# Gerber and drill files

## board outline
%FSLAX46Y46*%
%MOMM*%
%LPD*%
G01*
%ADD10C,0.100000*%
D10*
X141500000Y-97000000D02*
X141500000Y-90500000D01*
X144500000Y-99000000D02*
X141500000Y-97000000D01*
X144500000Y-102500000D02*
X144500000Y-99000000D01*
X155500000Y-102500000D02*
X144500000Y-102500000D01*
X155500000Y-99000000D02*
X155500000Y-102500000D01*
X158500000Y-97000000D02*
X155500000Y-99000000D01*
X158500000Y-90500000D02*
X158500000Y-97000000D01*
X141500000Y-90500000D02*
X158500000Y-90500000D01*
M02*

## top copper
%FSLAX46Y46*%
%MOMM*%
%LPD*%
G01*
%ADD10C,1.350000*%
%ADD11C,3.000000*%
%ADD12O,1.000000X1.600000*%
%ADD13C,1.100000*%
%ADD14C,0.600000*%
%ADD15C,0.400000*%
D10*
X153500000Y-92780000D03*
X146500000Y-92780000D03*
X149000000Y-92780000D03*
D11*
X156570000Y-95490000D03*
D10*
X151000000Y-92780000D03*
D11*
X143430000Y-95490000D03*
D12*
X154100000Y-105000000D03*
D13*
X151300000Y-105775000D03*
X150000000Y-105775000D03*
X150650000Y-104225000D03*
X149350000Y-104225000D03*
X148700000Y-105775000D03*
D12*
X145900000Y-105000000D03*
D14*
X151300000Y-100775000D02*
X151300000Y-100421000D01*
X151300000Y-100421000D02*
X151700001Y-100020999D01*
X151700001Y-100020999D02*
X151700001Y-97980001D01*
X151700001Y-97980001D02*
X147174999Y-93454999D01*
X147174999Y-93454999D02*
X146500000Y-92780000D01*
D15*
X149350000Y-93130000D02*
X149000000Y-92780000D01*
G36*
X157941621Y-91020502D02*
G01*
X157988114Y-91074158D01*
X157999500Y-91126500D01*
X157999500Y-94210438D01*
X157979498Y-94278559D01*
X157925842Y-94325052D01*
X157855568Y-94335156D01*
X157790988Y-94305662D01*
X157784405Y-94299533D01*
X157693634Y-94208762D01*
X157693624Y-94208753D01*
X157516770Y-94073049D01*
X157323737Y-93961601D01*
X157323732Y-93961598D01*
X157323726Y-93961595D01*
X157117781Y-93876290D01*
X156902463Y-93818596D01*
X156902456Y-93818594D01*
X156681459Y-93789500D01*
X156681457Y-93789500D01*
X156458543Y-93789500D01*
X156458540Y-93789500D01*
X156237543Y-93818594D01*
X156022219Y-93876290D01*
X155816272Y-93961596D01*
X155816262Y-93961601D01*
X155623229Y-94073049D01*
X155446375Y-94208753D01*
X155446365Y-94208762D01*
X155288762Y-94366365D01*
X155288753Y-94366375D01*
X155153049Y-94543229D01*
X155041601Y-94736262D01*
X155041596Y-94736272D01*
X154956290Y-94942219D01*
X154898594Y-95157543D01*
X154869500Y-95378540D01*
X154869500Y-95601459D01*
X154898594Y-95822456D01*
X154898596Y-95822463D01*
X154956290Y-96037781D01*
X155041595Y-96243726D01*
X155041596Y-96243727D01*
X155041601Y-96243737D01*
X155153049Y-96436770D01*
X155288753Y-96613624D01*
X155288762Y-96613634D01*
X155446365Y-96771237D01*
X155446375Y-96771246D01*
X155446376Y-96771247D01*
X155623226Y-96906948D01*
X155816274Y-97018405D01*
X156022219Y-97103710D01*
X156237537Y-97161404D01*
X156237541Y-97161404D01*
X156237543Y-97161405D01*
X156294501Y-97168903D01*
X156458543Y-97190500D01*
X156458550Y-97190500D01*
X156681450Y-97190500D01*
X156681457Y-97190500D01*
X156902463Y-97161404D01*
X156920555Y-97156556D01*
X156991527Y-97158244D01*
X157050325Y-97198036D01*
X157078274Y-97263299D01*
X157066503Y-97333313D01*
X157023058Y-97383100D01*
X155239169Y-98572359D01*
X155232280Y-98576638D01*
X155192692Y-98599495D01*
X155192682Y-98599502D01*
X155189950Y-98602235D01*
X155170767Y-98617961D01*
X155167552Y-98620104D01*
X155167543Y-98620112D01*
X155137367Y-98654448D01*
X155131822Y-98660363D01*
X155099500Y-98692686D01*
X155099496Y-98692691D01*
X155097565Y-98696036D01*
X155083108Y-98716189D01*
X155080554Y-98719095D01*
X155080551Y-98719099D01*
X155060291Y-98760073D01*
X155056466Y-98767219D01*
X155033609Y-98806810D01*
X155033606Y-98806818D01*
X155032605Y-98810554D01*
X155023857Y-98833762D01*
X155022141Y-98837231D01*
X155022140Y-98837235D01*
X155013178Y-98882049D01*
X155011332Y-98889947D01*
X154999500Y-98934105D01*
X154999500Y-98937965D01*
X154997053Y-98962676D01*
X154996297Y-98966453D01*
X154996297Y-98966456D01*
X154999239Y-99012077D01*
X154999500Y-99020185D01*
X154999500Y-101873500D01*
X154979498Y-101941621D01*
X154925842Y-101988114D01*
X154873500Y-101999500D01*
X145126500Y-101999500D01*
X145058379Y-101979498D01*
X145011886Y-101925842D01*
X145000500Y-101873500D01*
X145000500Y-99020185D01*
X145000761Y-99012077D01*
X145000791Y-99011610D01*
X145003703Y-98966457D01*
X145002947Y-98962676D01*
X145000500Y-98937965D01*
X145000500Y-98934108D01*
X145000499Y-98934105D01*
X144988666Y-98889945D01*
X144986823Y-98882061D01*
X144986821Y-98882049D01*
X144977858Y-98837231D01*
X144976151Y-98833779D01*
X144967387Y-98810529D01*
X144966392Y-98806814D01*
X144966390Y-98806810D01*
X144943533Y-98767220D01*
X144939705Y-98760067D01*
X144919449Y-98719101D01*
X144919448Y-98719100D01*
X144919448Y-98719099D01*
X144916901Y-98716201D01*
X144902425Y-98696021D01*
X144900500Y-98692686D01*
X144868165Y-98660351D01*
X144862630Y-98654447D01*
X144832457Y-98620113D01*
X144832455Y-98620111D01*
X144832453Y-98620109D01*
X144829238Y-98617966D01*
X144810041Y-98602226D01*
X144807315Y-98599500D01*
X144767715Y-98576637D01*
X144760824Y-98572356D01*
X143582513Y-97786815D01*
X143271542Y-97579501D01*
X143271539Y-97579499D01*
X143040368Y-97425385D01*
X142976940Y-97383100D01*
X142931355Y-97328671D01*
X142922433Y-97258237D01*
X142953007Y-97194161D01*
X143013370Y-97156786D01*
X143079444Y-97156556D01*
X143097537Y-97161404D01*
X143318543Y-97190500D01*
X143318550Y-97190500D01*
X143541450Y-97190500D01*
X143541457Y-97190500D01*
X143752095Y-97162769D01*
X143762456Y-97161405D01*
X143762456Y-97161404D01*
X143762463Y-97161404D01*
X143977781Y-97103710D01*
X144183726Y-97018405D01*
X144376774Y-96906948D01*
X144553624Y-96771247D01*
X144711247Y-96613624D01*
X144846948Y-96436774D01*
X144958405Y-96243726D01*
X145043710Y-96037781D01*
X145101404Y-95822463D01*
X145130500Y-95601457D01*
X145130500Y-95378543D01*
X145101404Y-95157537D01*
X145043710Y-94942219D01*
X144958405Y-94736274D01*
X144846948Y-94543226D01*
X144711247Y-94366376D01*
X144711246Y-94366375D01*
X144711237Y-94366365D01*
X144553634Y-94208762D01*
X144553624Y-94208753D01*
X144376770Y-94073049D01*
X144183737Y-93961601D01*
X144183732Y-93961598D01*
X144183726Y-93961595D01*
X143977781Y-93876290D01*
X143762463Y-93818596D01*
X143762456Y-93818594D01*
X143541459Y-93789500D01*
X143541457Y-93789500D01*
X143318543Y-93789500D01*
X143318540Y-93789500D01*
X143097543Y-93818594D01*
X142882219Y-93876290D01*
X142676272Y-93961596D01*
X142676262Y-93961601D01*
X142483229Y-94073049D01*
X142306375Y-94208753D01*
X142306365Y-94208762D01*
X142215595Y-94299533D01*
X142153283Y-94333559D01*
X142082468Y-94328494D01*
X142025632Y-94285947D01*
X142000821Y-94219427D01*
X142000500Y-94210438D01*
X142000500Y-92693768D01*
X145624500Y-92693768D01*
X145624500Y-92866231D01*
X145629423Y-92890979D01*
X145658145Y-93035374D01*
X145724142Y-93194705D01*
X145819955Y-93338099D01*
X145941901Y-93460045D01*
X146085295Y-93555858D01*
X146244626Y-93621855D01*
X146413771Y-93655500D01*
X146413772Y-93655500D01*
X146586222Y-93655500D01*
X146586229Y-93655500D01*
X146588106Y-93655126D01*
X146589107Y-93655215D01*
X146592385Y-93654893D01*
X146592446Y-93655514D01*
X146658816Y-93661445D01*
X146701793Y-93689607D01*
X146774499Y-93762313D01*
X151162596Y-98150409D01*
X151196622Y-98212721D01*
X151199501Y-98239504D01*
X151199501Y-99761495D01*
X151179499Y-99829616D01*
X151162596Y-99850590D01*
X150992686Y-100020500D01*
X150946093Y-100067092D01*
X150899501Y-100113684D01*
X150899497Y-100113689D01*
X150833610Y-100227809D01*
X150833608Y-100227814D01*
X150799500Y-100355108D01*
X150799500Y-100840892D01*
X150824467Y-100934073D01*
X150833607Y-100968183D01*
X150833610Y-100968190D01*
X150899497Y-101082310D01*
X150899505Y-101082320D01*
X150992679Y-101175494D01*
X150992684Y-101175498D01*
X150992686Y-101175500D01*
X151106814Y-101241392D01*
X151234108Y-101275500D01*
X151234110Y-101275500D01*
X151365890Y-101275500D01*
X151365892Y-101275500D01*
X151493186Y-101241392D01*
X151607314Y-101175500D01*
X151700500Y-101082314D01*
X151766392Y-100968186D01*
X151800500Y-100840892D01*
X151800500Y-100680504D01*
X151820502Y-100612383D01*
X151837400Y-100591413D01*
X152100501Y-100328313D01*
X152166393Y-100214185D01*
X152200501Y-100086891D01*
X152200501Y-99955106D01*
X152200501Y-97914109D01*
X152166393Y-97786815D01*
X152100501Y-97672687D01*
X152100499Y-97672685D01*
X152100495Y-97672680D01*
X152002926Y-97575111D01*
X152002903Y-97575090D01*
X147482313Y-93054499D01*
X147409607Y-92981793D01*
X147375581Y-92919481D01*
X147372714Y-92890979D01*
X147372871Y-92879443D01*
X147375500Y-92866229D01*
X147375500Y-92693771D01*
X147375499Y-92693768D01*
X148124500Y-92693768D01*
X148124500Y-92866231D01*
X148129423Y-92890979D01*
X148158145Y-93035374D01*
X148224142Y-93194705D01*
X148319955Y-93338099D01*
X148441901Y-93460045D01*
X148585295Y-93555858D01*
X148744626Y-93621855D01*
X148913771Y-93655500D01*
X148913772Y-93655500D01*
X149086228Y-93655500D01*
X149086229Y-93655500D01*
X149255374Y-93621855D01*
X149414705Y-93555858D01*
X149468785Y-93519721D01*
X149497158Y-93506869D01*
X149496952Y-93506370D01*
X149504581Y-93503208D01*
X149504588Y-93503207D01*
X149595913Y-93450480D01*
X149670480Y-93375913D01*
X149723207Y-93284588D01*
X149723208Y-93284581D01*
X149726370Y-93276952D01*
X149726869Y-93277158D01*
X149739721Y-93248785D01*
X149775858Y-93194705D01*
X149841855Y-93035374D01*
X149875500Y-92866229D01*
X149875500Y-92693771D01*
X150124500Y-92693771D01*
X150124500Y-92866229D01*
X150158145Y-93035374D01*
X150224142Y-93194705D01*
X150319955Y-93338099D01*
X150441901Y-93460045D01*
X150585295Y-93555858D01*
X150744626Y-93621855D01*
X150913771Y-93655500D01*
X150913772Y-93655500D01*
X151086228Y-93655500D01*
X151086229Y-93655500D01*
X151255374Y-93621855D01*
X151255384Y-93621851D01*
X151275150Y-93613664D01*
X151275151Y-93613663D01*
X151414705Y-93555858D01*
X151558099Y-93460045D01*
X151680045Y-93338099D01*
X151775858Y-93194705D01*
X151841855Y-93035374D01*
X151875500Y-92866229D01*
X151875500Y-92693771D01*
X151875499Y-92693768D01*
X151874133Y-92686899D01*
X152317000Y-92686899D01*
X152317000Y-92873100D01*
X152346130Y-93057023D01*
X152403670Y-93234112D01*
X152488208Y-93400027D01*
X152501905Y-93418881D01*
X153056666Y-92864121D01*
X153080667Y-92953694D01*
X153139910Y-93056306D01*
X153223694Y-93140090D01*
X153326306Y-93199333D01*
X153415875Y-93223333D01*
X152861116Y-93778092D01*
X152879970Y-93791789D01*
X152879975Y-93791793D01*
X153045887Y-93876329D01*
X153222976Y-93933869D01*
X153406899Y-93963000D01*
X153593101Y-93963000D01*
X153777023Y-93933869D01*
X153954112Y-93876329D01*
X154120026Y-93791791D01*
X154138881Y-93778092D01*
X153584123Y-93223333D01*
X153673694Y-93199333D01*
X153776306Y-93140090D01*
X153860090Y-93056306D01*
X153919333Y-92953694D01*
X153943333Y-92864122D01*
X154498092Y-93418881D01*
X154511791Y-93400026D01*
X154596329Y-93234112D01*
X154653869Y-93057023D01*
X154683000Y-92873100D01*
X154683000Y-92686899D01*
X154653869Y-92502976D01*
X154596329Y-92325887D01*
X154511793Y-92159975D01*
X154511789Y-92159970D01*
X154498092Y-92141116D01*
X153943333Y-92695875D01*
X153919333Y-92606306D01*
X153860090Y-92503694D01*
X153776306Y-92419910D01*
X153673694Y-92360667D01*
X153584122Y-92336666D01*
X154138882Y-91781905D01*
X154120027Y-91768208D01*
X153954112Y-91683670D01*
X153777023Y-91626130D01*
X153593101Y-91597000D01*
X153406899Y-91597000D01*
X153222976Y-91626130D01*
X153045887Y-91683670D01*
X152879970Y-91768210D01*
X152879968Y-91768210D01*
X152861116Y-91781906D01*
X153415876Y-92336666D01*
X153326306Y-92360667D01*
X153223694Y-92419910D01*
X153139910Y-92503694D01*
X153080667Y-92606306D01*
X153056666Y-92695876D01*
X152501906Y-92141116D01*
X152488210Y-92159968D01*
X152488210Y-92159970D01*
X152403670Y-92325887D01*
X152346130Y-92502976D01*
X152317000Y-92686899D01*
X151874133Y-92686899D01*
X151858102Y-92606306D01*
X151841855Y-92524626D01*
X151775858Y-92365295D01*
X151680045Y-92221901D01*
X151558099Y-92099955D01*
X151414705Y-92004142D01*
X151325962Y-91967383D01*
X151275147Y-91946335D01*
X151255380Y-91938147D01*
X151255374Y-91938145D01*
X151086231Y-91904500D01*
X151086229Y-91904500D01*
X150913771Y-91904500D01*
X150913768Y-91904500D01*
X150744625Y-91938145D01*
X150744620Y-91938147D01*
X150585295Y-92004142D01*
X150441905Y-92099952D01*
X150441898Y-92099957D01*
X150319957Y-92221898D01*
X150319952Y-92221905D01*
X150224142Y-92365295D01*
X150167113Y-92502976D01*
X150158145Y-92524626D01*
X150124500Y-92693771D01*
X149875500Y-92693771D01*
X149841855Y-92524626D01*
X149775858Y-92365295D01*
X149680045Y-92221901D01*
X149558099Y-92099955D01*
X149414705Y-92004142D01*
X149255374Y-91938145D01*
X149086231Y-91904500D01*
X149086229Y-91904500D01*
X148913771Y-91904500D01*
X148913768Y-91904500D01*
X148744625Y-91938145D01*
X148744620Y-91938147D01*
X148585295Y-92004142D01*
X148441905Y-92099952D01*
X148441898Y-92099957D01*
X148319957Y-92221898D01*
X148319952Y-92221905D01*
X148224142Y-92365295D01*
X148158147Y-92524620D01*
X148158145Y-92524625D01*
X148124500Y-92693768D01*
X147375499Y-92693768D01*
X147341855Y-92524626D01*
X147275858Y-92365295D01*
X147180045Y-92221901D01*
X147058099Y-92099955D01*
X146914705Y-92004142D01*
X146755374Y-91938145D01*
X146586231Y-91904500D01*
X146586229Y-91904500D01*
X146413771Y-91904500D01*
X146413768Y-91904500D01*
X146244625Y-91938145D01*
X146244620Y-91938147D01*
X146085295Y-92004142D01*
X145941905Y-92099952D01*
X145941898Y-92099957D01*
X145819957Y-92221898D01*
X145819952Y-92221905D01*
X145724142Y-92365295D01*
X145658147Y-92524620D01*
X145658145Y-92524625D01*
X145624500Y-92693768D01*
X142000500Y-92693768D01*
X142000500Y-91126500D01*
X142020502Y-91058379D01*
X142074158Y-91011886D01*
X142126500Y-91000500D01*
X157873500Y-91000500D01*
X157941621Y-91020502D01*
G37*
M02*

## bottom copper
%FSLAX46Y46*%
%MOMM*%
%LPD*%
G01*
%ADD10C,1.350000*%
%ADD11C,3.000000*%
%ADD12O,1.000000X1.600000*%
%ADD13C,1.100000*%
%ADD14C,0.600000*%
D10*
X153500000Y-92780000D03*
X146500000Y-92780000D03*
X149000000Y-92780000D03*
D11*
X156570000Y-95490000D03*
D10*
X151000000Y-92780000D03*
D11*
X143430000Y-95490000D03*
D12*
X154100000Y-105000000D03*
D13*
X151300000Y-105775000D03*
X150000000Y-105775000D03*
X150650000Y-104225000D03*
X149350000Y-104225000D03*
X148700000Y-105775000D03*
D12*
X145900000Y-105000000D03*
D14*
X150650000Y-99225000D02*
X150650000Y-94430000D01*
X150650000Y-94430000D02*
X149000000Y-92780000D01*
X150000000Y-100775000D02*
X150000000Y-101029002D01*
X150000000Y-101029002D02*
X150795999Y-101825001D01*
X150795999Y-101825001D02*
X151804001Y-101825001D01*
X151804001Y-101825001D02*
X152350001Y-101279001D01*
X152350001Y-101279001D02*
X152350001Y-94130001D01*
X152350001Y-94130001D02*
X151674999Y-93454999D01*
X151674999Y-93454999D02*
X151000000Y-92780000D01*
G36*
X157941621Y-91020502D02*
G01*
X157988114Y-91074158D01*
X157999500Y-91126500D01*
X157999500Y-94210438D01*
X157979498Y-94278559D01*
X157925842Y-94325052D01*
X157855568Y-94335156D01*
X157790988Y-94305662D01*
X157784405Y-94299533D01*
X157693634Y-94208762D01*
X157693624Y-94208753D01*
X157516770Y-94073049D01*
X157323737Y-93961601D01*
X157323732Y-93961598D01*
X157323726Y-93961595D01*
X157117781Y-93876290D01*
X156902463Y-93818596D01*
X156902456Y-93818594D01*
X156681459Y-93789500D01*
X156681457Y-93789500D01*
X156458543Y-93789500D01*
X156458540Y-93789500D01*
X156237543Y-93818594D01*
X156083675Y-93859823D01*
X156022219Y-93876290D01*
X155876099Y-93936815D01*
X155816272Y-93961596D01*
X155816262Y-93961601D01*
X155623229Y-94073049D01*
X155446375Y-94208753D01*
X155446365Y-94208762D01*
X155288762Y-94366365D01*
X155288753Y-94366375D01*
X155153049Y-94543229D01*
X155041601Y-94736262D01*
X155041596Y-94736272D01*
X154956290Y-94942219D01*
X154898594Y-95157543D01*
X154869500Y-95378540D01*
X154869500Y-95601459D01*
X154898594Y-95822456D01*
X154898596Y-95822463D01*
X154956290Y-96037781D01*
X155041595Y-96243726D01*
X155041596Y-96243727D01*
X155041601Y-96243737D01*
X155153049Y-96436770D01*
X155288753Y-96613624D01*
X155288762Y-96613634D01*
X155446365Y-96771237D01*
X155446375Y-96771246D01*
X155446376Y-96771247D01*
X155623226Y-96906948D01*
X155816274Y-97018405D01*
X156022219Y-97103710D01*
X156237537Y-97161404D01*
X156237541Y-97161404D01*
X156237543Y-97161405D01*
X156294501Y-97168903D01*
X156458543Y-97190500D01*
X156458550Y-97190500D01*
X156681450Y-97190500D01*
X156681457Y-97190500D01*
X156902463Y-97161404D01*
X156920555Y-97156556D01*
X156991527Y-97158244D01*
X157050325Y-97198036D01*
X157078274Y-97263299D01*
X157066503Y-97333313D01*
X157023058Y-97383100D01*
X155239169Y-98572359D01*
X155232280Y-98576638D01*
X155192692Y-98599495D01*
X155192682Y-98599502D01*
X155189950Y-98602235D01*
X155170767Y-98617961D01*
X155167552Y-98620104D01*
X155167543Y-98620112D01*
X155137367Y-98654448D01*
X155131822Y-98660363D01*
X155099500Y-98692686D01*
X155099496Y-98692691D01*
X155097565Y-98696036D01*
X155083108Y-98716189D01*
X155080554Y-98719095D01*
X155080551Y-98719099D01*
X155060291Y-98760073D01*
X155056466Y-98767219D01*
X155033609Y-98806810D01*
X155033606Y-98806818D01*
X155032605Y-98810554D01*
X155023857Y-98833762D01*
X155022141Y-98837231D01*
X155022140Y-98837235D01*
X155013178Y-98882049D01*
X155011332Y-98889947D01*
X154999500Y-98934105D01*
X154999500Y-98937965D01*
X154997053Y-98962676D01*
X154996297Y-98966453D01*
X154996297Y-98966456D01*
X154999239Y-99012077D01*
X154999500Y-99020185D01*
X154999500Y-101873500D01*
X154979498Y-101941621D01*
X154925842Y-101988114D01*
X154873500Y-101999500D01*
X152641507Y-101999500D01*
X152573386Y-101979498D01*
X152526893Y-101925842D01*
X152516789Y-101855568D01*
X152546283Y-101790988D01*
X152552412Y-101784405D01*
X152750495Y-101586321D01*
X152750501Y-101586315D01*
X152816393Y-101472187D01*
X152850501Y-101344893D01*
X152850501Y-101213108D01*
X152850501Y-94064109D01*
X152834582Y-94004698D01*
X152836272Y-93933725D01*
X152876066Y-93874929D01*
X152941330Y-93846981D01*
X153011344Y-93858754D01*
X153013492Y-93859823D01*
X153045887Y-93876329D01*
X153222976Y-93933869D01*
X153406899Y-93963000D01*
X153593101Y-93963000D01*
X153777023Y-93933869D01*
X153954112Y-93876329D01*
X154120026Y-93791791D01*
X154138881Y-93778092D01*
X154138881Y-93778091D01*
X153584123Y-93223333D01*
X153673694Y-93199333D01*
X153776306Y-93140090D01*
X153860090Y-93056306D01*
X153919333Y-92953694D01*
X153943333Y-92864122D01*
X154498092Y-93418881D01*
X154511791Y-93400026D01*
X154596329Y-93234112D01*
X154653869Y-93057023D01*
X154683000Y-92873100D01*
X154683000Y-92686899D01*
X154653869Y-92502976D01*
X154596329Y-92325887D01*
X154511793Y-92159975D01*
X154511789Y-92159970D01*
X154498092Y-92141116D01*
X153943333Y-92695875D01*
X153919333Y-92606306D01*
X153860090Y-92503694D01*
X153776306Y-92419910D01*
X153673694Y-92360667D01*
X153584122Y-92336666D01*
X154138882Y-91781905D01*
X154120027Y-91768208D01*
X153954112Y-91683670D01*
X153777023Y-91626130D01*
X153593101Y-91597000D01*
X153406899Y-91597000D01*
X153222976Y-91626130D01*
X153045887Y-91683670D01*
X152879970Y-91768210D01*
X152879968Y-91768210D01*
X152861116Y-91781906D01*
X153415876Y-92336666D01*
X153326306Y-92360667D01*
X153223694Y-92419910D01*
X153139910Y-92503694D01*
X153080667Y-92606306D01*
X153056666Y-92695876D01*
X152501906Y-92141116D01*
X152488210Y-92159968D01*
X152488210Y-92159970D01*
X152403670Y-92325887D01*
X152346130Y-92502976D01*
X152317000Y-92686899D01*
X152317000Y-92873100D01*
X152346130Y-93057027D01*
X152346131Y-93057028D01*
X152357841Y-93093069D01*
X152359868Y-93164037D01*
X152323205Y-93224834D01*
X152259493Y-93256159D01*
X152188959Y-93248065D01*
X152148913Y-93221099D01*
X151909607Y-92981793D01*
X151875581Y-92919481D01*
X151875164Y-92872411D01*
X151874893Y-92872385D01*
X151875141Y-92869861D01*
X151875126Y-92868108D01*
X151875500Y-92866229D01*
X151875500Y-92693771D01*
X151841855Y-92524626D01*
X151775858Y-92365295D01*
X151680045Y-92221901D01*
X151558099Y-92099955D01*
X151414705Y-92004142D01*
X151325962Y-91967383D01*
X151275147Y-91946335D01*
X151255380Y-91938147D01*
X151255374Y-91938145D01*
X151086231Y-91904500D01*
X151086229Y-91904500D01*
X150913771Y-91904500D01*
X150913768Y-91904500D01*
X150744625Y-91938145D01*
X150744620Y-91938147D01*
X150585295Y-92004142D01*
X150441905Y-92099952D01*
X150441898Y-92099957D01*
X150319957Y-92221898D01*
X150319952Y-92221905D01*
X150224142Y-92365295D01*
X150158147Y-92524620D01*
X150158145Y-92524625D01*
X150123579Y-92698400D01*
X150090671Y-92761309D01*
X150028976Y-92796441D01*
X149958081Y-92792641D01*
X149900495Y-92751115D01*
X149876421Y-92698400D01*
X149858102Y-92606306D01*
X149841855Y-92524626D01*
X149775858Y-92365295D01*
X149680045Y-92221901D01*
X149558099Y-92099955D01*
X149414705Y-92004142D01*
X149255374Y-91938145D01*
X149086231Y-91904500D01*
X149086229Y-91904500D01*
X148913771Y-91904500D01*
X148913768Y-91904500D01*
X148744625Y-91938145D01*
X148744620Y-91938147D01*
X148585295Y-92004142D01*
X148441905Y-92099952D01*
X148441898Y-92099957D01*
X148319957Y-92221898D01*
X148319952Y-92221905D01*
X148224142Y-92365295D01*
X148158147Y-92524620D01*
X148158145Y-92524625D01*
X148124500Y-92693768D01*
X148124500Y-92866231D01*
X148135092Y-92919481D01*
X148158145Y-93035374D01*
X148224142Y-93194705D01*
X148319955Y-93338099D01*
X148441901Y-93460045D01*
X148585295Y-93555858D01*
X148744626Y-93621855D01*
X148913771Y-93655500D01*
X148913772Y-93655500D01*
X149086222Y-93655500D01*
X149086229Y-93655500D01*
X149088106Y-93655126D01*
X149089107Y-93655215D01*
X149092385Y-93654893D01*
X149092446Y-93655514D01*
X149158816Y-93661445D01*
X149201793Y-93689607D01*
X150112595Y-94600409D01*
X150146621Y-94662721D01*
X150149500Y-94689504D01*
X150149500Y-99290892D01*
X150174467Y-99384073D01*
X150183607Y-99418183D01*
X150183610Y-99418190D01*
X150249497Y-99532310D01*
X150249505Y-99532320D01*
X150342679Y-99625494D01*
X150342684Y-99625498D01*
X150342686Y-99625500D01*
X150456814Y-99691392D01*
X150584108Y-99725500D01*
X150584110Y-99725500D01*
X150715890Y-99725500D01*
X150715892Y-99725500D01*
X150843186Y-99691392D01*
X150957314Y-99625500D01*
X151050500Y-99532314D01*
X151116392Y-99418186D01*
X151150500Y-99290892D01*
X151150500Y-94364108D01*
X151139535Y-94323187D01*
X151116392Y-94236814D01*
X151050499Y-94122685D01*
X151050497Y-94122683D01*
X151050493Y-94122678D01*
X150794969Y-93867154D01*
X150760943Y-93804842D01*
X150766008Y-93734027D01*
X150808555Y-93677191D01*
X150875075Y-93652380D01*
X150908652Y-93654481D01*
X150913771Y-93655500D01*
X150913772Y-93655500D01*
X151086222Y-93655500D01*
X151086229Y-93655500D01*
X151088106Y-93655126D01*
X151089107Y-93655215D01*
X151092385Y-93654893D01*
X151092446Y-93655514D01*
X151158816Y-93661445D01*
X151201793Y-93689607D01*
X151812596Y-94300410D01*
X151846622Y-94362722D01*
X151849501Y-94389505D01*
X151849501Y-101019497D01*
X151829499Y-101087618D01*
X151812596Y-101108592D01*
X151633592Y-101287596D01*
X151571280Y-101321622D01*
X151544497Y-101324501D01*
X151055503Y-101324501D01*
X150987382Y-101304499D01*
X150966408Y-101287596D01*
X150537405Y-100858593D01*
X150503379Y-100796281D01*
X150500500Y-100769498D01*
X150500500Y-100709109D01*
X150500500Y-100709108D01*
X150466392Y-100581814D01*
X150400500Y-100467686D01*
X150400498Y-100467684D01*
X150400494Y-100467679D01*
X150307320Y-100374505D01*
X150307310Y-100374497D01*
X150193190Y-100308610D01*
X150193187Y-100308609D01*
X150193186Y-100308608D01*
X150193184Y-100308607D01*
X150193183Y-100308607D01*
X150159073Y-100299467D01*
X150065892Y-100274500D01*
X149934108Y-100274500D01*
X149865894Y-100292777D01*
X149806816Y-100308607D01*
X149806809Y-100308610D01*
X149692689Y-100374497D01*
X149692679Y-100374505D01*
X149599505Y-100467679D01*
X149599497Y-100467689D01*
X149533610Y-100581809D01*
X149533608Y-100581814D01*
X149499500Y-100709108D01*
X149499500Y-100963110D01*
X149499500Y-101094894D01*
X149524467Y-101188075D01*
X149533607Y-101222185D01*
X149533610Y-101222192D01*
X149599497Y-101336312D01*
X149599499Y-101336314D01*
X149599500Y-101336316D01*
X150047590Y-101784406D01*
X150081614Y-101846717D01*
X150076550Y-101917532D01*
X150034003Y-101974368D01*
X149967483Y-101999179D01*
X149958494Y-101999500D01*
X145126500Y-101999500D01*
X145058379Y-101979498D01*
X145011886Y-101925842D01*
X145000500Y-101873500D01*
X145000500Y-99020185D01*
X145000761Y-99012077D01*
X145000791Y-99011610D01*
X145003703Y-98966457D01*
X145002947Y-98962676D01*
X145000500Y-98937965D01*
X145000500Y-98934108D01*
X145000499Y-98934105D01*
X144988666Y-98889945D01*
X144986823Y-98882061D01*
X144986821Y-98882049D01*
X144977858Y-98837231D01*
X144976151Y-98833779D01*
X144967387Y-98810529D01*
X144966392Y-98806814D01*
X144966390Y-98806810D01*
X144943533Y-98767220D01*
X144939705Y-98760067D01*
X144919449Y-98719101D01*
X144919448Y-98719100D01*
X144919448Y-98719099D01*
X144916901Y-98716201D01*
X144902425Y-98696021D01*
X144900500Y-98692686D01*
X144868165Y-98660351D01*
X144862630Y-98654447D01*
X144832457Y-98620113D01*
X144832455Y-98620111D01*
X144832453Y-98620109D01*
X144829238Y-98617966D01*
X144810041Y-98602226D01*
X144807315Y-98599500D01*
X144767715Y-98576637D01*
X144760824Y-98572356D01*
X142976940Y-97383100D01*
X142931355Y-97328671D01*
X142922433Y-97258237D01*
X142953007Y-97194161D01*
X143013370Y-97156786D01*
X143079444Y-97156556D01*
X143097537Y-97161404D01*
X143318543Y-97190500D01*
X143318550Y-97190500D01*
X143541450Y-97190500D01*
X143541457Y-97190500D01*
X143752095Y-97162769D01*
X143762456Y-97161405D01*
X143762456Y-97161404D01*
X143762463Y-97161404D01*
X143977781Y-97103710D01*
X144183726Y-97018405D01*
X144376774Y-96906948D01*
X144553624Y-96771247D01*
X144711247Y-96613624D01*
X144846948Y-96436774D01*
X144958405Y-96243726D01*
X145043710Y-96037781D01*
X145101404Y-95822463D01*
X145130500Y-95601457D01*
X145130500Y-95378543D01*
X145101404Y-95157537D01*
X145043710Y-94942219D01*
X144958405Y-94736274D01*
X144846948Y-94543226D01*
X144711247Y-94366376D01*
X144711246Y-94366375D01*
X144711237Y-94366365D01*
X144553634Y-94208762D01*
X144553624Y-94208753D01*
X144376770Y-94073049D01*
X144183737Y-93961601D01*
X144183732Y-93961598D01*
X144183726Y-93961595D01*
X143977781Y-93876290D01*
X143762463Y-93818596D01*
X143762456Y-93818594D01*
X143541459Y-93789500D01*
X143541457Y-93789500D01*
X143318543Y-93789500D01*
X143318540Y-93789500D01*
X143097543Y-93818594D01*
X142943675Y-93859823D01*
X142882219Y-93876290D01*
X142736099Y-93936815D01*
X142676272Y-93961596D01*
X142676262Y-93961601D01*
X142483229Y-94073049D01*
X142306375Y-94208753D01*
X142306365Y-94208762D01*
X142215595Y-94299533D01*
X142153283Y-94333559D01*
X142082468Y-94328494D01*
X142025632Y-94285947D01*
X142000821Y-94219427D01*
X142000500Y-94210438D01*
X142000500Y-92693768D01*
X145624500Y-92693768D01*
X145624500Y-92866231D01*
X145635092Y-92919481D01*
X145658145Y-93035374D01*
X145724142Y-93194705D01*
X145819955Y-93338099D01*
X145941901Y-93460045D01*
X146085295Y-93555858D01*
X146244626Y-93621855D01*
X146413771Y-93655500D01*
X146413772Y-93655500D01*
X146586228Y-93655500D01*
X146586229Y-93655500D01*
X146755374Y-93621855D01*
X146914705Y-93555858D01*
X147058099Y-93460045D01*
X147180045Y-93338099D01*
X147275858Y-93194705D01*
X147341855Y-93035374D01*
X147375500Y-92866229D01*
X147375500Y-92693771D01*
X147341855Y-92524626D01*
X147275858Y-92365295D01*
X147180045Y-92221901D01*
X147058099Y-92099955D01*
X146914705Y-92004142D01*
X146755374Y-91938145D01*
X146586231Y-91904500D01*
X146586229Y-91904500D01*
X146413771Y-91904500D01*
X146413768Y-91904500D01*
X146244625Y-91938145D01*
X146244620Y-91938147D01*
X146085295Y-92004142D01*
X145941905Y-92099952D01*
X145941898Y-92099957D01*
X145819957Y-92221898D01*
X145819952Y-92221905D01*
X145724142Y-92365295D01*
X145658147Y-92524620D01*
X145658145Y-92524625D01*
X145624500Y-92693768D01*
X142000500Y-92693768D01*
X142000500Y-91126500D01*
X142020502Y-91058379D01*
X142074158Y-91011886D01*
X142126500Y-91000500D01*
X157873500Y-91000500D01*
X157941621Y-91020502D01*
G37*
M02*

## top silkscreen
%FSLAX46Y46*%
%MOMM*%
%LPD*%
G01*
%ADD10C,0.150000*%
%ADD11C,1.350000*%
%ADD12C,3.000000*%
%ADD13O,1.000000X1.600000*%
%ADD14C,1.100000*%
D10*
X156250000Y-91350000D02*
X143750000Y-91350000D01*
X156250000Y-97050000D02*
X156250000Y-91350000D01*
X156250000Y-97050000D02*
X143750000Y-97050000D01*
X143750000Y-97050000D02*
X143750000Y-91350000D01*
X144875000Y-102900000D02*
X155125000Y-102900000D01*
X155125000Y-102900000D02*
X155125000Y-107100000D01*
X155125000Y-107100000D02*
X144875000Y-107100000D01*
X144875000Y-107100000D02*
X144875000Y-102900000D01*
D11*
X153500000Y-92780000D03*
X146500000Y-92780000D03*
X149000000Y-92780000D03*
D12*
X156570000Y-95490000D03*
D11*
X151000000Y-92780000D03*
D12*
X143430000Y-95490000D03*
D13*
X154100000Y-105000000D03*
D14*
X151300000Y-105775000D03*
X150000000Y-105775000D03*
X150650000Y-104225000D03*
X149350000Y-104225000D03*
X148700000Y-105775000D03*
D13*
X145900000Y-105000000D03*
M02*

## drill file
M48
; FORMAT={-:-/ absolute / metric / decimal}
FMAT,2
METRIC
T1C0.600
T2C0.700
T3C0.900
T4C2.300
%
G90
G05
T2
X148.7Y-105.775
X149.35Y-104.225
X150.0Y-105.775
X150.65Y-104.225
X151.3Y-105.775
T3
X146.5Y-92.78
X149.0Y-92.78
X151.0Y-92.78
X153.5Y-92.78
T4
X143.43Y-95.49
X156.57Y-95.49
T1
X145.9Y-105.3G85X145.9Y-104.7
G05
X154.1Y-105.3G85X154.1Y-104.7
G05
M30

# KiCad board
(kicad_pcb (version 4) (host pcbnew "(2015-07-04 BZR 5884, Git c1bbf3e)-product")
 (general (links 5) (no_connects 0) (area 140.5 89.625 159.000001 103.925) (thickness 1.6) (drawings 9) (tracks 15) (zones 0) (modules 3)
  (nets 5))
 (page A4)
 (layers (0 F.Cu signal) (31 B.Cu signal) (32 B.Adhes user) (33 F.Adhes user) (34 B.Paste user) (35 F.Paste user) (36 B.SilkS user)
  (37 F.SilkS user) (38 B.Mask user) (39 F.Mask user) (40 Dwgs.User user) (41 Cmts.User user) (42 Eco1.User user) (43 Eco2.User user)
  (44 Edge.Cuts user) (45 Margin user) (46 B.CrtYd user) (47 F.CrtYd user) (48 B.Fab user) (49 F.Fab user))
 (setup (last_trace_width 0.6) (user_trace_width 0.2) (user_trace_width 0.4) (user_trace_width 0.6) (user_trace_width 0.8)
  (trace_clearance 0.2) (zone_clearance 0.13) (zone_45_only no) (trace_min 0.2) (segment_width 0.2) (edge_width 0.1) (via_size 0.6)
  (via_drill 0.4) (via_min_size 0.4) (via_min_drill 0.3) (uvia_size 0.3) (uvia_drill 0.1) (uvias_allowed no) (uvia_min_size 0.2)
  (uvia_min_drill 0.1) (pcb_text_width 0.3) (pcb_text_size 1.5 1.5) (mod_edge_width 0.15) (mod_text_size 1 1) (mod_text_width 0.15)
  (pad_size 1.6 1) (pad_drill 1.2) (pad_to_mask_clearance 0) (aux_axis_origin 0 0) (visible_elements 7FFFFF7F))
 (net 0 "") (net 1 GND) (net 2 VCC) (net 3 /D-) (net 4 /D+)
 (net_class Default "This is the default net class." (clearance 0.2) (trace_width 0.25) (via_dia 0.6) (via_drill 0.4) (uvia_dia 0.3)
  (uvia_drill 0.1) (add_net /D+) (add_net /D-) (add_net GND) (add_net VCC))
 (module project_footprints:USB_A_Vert (layer F.Cu) (at 150 97)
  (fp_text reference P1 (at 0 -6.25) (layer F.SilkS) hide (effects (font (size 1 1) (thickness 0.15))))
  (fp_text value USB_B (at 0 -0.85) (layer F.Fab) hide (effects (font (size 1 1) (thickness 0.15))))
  (fp_line (start 6.25 -5.65) (end -6.25 -5.65) (layer F.SilkS) (width 0.15))
  (fp_line (start 6.25 0.05) (end 6.25 -5.65) (layer F.SilkS) (width 0.15))
  (fp_line (start 6.25 0.05) (end -6.25 0.05) (layer F.SilkS) (width 0.15))
  (fp_line (start -6.25 0.05) (end -6.25 -5.65) (layer F.SilkS) (width 0.15))
  (pad 4 thru_hole circle (at 3.5 -4.22 90) (size 1.35 1.35) (drill 0.9) (layers *.Cu *.Mask F.SilkS) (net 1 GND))
  (pad 1 thru_hole circle (at -3.5 -4.22 90) (size 1.35 1.35) (drill 0.9) (layers *.Cu *.Mask F.SilkS) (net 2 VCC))
  (pad 2 thru_hole circle (at -1 -4.22 90) (size 1.35 1.35) (drill 0.9) (layers *.Cu *.Mask F.SilkS) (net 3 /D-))
  (pad 6 thru_hole circle (at 6.57 -1.51 90) (size 3 3) (drill 2.3) (layers *.Cu *.Mask F.SilkS))
  (pad 3 thru_hole circle (at 1 -4.22 90) (size 1.35 1.35) (drill 0.9) (layers *.Cu *.Mask F.SilkS) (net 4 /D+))
  (pad 6 thru_hole circle (at -6.57 -1.51 90) (size 3 3) (drill 2.3) (layers *.Cu *.Mask F.SilkS)))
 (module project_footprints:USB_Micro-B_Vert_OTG (layer F.Cu) (at 150 105)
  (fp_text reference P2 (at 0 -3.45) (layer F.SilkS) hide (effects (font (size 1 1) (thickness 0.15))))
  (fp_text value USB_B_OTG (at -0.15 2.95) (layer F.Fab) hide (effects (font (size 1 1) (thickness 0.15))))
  (fp_line (start -5.125 -2.1) (end 5.125 -2.1) (layer F.SilkS) (width 0.15))
  (fp_line (start 5.125 -2.1) (end 5.125 2.1) (layer F.SilkS) (width 0.15))
  (fp_line (start 5.125 2.1) (end -5.125 2.1) (layer F.SilkS) (width 0.15))
  (fp_line (start -5.125 2.1) (end -5.125 -2.1) (layer F.SilkS) (width 0.15))
  (pad 6 thru_hole oval (at 4.1 0 90) (size 1.6 1) (drill oval 1.2 0.6) (layers *.Cu *.Mask F.SilkS))
  (pad 1 thru_hole circle (at 1.3 0.775 90) (size 1.1 1.1) (drill 0.7) (layers *.Cu *.Mask F.SilkS) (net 2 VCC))
  (pad 3 thru_hole circle (at 0 0.775 90) (size 1.1 1.1) (drill 0.7) (layers *.Cu *.Mask F.SilkS) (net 4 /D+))
  (pad 2 thru_hole circle (at 0.65 -0.775 90) (size 1.1 1.1) (drill 0.7) (layers *.Cu *.Mask F.SilkS) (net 3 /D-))
  (pad 4 thru_hole circle (at -0.65 -0.775 90) (size 1.1 1.1) (drill 0.7) (layers *.Cu *.Mask F.SilkS) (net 1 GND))
  (pad 5 thru_hole circle (at -1.3 0.775 90) (size 1.1 1.1) (drill 0.7) (layers *.Cu *.Mask F.SilkS) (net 1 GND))
  (pad 6 thru_hole oval (at -4.1 0 90) (size 1.6 1) (drill oval 1.2 0.6) (layers *.Cu *.Mask F.SilkS)))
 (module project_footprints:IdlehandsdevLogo (layer B.Cu) (at 150 96)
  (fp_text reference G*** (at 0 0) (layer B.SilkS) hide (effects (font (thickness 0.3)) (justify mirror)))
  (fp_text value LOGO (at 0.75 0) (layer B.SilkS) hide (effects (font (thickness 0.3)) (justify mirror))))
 (gr_line (start 141.5 97) (end 141.5 90.5) (layer Edge.Cuts) (width 0.1))
 (gr_line (start 144.5 99) (end 141.5 97) (layer Edge.Cuts) (width 0.1))
 (gr_line (start 144.5 102.5) (end 144.5 99) (layer Edge.Cuts) (width 0.1))
 (gr_line (start 155.5 102.5) (end 144.5 102.5) (layer Edge.Cuts) (width 0.1))
 (gr_line (start 155.5 99) (end 155.5 102.5) (layer Edge.Cuts) (width 0.1))
 (gr_line (start 158.5 97) (end 155.5 99) (layer Edge.Cuts) (width 0.1))
 (gr_line (start 158.5 90.5) (end 158.5 97) (layer Edge.Cuts) (width 0.1))
 (gr_line (start 141.5 90.5) (end 158.5 90.5) (layer Edge.Cuts) (width 0.1))
 (segment (start 151.3 100.775) (end 151.3 100.421) (width 0.6) (layer F.Cu) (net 2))
 (segment (start 151.3 100.421) (end 151.700001 100.020999) (width 0.6) (layer F.Cu) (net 2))
 (segment (start 151.700001 100.020999) (end 151.700001 97.980001) (width 0.6) (layer F.Cu) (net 2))
 (segment (start 151.700001 97.980001) (end 147.174999 93.454999) (width 0.6) (layer F.Cu) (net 2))
 (segment (start 147.174999 93.454999) (end 146.5 92.78) (width 0.6) (layer F.Cu) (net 2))
 (segment (start 150.65 99.225) (end 150.65 94.43) (width 0.6) (layer B.Cu) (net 3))
 (segment (start 150.65 94.43) (end 149 92.78) (width 0.6) (layer B.Cu) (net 3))
 (segment (start 149.35 93.13) (end 149 92.78) (width 0.4) (layer F.Cu) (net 3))
 (segment (start 150 100.775) (end 150 101.029002) (width 0.6) (layer B.Cu) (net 4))
 (segment (start 150 101.029002) (end 150.795999 101.825001) (width 0.6) (layer B.Cu) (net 4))
 (segment (start 150.795999 101.825001) (end 151.804001 101.825001) (width 0.6) (layer B.Cu) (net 4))
 (segment (start 151.804001 101.825001) (end 152.350001 101.279001) (width 0.6) (layer B.Cu) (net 4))
 (segment (start 152.350001 101.279001) (end 152.350001 94.130001) (width 0.6) (layer B.Cu) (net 4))
 (segment (start 152.350001 94.130001) (end 151.674999 93.454999) (width 0.6) (layer B.Cu) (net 4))
 (segment (start 151.674999 93.454999) (end 151 92.78) (width 0.6) (layer B.Cu) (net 4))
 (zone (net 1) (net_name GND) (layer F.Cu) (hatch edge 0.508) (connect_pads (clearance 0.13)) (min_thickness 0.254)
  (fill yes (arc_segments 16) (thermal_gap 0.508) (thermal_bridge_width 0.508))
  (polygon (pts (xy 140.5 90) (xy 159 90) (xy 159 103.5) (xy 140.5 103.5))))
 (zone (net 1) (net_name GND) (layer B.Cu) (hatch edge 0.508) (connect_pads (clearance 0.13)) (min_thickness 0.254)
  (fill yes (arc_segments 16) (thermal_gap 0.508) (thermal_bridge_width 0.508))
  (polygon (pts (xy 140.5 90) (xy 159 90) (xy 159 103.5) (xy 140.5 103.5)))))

